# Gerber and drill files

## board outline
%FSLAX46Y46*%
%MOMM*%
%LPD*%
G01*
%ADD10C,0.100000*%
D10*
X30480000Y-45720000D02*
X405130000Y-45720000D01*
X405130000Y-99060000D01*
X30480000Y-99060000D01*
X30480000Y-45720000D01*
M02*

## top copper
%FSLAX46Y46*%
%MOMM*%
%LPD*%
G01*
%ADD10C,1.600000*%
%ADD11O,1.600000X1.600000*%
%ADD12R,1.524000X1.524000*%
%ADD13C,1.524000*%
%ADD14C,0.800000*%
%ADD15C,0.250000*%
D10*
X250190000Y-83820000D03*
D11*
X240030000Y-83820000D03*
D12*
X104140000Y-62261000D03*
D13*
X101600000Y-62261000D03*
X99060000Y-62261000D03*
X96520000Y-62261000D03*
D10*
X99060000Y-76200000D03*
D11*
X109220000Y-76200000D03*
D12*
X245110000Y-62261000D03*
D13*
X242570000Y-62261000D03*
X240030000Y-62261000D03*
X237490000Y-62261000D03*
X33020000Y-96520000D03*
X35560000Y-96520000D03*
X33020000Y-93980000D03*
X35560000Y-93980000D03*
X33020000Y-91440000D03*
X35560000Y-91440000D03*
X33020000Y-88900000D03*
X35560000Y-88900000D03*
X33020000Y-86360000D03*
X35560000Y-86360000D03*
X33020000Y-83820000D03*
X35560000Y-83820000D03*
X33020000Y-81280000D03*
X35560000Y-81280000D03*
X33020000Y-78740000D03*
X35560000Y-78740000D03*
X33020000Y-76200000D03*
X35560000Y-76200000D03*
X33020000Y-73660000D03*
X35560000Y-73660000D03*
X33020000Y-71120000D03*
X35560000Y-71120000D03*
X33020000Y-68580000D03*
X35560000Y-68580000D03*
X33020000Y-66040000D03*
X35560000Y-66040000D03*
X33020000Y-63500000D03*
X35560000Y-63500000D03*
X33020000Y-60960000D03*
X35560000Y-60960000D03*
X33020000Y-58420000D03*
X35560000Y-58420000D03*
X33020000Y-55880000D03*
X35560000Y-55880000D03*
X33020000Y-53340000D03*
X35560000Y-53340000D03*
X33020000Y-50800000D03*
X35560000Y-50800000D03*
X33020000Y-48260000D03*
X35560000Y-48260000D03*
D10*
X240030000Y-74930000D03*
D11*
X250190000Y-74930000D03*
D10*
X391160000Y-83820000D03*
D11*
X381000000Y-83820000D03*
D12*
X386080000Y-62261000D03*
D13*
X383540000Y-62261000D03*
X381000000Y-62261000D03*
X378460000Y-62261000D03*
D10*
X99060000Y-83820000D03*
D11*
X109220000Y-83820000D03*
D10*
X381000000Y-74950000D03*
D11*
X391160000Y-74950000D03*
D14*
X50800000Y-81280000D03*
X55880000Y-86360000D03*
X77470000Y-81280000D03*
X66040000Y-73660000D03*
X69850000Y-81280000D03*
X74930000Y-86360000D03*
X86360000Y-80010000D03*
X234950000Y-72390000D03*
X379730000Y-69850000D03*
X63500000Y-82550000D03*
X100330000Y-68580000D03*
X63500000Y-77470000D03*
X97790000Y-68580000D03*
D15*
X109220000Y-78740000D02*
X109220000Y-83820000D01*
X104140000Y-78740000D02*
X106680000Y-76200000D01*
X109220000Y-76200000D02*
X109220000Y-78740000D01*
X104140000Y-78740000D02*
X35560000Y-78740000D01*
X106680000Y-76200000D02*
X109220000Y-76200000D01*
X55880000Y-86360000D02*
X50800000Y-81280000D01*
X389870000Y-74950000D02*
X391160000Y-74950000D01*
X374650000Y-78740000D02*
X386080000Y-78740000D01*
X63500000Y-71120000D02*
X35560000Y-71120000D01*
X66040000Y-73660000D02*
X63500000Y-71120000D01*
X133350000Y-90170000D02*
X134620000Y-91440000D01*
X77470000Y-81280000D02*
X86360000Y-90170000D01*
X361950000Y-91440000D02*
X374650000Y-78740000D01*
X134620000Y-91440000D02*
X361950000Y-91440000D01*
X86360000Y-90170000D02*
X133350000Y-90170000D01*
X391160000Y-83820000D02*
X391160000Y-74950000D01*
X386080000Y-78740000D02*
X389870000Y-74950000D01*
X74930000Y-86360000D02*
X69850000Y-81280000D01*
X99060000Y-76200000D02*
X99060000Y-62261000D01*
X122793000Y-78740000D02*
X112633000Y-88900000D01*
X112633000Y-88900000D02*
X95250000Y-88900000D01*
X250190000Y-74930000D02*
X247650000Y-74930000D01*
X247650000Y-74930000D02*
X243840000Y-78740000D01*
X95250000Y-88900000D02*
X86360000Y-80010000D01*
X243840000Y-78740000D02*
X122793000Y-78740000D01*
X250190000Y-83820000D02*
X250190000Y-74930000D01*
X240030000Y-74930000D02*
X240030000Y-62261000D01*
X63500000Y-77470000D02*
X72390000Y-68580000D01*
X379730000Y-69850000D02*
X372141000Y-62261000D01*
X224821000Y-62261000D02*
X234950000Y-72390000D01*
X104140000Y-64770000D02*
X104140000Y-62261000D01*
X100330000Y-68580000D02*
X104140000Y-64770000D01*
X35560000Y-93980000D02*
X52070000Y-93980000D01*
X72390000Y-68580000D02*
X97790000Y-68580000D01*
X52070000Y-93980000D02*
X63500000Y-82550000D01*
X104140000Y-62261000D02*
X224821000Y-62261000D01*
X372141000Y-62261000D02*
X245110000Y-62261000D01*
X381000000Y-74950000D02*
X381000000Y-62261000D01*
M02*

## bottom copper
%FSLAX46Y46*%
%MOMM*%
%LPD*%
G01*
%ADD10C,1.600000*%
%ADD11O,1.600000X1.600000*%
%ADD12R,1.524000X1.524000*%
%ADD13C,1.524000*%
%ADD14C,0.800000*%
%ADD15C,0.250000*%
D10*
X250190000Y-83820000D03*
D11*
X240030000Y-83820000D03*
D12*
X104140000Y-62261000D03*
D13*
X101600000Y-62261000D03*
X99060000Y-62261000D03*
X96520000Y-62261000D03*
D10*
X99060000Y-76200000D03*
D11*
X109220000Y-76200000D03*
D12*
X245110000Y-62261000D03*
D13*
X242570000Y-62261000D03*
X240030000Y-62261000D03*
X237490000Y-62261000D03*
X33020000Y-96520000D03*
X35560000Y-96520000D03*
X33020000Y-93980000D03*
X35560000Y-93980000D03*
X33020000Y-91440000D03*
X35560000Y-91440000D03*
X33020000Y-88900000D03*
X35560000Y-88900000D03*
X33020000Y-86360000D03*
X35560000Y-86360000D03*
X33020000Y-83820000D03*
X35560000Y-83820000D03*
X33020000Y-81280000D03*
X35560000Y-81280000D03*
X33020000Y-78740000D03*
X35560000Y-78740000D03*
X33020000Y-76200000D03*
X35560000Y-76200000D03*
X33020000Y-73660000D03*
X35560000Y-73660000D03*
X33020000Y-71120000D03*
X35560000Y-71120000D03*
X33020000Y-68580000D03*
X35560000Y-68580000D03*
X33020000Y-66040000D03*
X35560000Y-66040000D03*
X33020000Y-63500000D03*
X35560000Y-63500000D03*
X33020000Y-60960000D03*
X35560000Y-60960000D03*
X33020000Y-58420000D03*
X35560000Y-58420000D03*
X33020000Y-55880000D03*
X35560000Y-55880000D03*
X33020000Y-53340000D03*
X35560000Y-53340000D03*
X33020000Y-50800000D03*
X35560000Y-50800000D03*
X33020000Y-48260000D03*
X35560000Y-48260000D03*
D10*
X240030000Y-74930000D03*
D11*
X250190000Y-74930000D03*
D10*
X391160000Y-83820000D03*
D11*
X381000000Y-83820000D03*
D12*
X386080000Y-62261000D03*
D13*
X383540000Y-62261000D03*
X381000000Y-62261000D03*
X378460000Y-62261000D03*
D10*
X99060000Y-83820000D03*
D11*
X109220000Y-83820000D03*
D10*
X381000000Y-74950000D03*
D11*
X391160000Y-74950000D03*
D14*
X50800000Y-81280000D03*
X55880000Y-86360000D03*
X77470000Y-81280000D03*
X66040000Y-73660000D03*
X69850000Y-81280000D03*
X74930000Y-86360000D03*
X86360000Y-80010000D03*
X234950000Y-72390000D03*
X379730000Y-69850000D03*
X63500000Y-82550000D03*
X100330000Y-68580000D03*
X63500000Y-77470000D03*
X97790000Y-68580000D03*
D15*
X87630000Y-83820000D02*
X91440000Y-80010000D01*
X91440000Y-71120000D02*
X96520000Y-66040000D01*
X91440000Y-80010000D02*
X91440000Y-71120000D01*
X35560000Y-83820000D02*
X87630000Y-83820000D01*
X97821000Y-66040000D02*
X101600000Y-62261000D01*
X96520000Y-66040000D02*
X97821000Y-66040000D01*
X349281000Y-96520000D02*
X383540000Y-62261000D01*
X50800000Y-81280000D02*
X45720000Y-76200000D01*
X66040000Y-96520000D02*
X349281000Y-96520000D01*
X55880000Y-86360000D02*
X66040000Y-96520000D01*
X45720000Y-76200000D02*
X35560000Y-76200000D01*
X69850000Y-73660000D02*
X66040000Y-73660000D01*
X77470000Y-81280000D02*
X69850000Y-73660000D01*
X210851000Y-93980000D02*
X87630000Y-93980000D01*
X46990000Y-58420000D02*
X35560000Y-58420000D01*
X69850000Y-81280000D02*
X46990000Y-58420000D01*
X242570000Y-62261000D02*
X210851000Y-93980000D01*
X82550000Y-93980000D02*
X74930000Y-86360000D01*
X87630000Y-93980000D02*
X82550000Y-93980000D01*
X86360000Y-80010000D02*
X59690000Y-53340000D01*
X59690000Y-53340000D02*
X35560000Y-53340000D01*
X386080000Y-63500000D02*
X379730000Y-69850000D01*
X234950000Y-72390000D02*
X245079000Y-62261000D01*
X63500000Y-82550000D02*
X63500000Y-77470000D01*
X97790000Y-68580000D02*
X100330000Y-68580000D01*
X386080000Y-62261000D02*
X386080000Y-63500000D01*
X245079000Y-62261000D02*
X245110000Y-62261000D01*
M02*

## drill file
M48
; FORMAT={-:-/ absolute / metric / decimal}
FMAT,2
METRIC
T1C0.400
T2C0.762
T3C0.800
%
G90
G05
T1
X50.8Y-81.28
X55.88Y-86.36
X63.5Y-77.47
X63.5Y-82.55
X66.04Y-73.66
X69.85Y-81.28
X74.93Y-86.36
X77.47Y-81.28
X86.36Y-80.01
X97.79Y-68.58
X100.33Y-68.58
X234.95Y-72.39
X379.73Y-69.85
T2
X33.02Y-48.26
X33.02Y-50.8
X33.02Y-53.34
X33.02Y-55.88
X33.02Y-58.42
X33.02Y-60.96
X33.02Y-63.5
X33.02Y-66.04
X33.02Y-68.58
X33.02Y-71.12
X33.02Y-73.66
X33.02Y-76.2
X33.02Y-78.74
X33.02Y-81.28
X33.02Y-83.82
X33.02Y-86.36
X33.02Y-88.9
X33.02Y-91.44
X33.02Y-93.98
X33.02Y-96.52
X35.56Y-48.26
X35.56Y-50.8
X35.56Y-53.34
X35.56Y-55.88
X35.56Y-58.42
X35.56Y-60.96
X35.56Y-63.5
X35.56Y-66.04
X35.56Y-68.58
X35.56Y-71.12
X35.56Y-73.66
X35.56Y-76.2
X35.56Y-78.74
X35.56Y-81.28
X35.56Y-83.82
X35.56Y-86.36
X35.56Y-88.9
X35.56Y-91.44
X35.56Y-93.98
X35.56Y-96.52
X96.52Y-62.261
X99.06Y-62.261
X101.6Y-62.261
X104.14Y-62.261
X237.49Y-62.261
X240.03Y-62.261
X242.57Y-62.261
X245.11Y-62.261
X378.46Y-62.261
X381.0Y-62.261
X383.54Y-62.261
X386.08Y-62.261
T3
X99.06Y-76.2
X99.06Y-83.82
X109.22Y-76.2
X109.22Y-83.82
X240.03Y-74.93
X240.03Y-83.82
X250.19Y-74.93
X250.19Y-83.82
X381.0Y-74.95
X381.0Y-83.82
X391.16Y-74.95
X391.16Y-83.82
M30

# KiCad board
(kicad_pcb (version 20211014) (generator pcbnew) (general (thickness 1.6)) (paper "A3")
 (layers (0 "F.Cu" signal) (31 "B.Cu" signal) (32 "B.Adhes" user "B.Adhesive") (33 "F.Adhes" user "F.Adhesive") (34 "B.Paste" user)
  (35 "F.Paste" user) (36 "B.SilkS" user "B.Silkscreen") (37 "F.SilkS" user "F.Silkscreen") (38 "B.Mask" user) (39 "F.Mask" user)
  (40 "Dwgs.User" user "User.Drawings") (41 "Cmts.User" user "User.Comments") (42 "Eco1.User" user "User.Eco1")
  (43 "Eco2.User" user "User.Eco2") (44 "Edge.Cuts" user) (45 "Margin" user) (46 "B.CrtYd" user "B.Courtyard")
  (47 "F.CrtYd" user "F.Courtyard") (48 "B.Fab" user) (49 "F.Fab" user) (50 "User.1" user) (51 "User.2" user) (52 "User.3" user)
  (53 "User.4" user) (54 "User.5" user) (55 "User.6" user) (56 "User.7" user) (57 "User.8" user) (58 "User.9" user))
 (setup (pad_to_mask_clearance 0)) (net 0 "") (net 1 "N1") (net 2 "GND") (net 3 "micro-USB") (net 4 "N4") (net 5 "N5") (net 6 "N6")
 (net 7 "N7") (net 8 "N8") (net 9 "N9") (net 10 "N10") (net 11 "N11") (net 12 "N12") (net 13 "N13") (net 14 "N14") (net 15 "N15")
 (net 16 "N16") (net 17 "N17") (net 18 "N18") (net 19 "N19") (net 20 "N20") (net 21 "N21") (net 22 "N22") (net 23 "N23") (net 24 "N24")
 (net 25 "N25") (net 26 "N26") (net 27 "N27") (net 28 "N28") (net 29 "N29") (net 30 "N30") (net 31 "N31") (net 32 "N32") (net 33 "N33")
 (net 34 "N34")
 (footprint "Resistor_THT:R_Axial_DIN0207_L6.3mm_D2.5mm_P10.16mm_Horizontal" (layer "F.Cu") (at 250.19 83.82 180)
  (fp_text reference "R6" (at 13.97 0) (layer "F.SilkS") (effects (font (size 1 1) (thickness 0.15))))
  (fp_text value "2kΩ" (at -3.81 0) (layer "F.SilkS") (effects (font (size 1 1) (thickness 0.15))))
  (pad "1" thru_hole circle (at 0 0 180) (size 1.6 1.6) (drill 0.8) (layers *.Cu *.Mask) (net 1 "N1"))
  (pad "2" thru_hole oval (at 10.16 0 180) (size 1.6 1.6) (drill 0.8) (layers *.Cu *.Mask) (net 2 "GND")))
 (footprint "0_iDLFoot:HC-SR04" (layer "F.Cu") (at 104.14 62.261 180)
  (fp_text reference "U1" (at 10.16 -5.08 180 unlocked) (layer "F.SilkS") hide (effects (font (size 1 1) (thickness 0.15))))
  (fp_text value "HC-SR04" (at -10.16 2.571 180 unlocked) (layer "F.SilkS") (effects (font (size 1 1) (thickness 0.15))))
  (pad "1" thru_hole rect (at 0 0 180) (size 1.524 1.524) (drill 0.762) (layers *.Cu *.Mask) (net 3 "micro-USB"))
  (pad "2" thru_hole circle (at 2.54 0 180) (size 1.524 1.524) (drill 0.762) (layers *.Cu *.Mask) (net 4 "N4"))
  (pad "3" thru_hole circle (at 5.08 0 180) (size 1.524 1.524) (drill 0.762) (layers *.Cu *.Mask) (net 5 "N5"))
  (pad "4" thru_hole circle (at 7.62 0 180) (size 1.524 1.524) (drill 0.762) (layers *.Cu *.Mask) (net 2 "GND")))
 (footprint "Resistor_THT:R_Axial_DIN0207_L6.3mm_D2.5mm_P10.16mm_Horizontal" (layer "F.Cu") (at 99.06 76.2)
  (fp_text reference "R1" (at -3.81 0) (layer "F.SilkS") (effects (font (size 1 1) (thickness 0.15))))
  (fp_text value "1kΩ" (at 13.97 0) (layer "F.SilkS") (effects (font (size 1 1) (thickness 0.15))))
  (pad "1" thru_hole circle (at 0 0) (size 1.6 1.6) (drill 0.8) (layers *.Cu *.Mask) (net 5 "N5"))
  (pad "2" thru_hole oval (at 10.16 0) (size 1.6 1.6) (drill 0.8) (layers *.Cu *.Mask) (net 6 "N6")))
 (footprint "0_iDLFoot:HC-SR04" (layer "F.Cu") (at 245.11 62.261 180)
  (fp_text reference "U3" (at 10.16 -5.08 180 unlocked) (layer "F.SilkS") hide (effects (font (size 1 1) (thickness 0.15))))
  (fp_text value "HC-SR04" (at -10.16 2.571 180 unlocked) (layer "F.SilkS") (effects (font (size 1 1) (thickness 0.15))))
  (pad "1" thru_hole rect (at 0 0 180) (size 1.524 1.524) (drill 0.762) (layers *.Cu *.Mask) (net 3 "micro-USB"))
  (pad "2" thru_hole circle (at 2.54 0 180) (size 1.524 1.524) (drill 0.762) (layers *.Cu *.Mask) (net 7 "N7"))
  (pad "3" thru_hole circle (at 5.08 0 180) (size 1.524 1.524) (drill 0.762) (layers *.Cu *.Mask) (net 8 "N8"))
  (pad "4" thru_hole circle (at 7.62 0 180) (size 1.524 1.524) (drill 0.762) (layers *.Cu *.Mask) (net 2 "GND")))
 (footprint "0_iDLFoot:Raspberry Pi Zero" (layer "F.Cu") (at 33.02 96.52)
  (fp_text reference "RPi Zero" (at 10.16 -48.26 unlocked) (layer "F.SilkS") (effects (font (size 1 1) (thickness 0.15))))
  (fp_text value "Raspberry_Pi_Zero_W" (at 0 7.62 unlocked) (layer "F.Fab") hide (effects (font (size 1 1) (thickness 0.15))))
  (pad "1" thru_hole circle (at 0 0) (size 1.524 1.524) (drill 0.762) (layers *.Cu *.Mask) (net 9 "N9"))
  (pad "2" thru_hole circle (at 2.54 0) (size 1.524 1.524) (drill 0.762) (layers *.Cu *.Mask))
  (pad "3" thru_hole circle (at 0 -2.54) (size 1.524 1.524) (drill 0.762) (layers *.Cu *.Mask) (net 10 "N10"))
  (pad "4" thru_hole circle (at 2.54 -2.54) (size 1.524 1.524) (drill 0.762) (layers *.Cu *.Mask) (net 3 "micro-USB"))
  (pad "5" thru_hole circle (at 0 -5.08) (size 1.524 1.524) (drill 0.762) (layers *.Cu *.Mask) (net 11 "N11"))
  (pad "6" thru_hole circle (at 2.54 -5.08) (size 1.524 1.524) (drill 0.762) (layers *.Cu *.Mask))
  (pad "7" thru_hole circle (at 0 -7.62) (size 1.524 1.524) (drill 0.762) (layers *.Cu *.Mask) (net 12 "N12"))
  (pad "8" thru_hole circle (at 2.54 -7.62) (size 1.524 1.524) (drill 0.762) (layers *.Cu *.Mask) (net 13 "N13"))
  (pad "9" thru_hole circle (at 0 -10.16) (size 1.524 1.524) (drill 0.762) (layers *.Cu *.Mask))
  (pad "10" thru_hole circle (at 2.54 -10.16) (size 1.524 1.524) (drill 0.762) (layers *.Cu *.Mask) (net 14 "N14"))
  (pad "11" thru_hole circle (at 0 -12.7) (size 1.524 1.524) (drill 0.762) (layers *.Cu *.Mask) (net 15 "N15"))
  (pad "12" thru_hole circle (at 2.54 -12.7) (size 1.524 1.524) (drill 0.762) (layers *.Cu *.Mask) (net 4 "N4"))
  (pad "13" thru_hole circle (at 0 -15.24) (size 1.524 1.524) (drill 0.762) (layers *.Cu *.Mask) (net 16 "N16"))
  (pad "14" thru_hole circle (at 2.54 -15.24) (size 1.524 1.524) (drill 0.762) (layers *.Cu *.Mask) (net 2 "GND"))
  (pad "15" thru_hole circle (at 0 -17.78) (size 1.524 1.524) (drill 0.762) (layers *.Cu *.Mask) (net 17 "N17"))
  (pad "16" thru_hole circle (at 2.54 -17.78) (size 1.524 1.524) (drill 0.762) (layers *.Cu *.Mask) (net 6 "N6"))
  (pad "17" thru_hole circle (at 0 -20.32) (size 1.524 1.524) (drill 0.762) (layers *.Cu *.Mask))
  (pad "18" thru_hole circle (at 2.54 -20.32) (size 1.524 1.524) (drill 0.762) (layers *.Cu *.Mask) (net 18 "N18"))
  (pad "19" thru_hole circle (at 0 -22.86) (size 1.524 1.524) (drill 0.762) (layers *.Cu *.Mask) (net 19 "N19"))
  (pad "20" thru_hole circle (at 2.54 -22.86) (size 1.524 1.524) (drill 0.762) (layers *.Cu *.Mask))
  (pad "21" thru_hole circle (at 0 -25.4) (size 1.524 1.524) (drill 0.762) (layers *.Cu *.Mask) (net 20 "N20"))
  (pad "22" thru_hole circle (at 2.54 -25.4) (size 1.524 1.524) (drill 0.762) (layers *.Cu *.Mask) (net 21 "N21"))
  (pad "23" thru_hole circle (at 0 -27.94) (size 1.524 1.524) (drill 0.762) (layers *.Cu *.Mask) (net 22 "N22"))
  (pad "24" thru_hole circle (at 2.54 -27.94) (size 1.524 1.524) (drill 0.762) (layers *.Cu *.Mask) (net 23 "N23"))
  (pad "25" thru_hole circle (at 0 -30.48) (size 1.524 1.524) (drill 0.762) (layers *.Cu *.Mask))
  (pad "26" thru_hole circle (at 2.54 -30.48) (size 1.524 1.524) (drill 0.762) (layers *.Cu *.Mask) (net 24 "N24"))
  (pad "27" thru_hole circle (at 0 -33.02) (size 1.524 1.524) (drill 0.762) (layers *.Cu *.Mask) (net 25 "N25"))
  (pad "28" thru_hole circle (at 2.54 -33.02) (size 1.524 1.524) (drill 0.762) (layers *.Cu *.Mask) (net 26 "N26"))
  (pad "29" thru_hole circle (at 0 -35.56) (size 1.524 1.524) (drill 0.762) (layers *.Cu *.Mask) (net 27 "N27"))
  (pad "30" thru_hole circle (at 2.54 -35.56) (size 1.524 1.524) (drill 0.762) (layers *.Cu *.Mask))
  (pad "31" thru_hole circle (at 0 -38.1) (size 1.524 1.524) (drill 0.762) (layers *.Cu *.Mask) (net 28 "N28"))
  (pad "32" thru_hole circle (at 2.54 -38.1) (size 1.524 1.524) (drill 0.762) (layers *.Cu *.Mask) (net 7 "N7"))
  (pad "33" thru_hole circle (at 0 -40.64) (size 1.524 1.524) (drill 0.762) (layers *.Cu *.Mask) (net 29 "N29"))
  (pad "34" thru_hole circle (at 2.54 -40.64) (size 1.524 1.524) (drill 0.762) (layers *.Cu *.Mask))
  (pad "35" thru_hole circle (at 0 -43.18) (size 1.524 1.524) (drill 0.762) (layers *.Cu *.Mask) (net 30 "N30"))
  (pad "36" thru_hole circle (at 2.54 -43.18) (size 1.524 1.524) (drill 0.762) (layers *.Cu *.Mask) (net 1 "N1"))
  (pad "37" thru_hole circle (at 0 -45.72) (size 1.524 1.524) (drill 0.762) (layers *.Cu *.Mask) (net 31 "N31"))
  (pad "38" thru_hole circle (at 2.54 -45.72) (size 1.524 1.524) (drill 0.762) (layers *.Cu *.Mask) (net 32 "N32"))
  (pad "39" thru_hole circle (at 0 -48.26) (size 1.524 1.524) (drill 0.762) (layers *.Cu *.Mask))
  (pad "40" thru_hole circle (at 2.54 -48.26) (size 1.524 1.524) (drill 0.762) (layers *.Cu *.Mask) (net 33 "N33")))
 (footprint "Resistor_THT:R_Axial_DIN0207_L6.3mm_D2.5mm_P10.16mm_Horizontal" (layer "F.Cu") (at 240.03 74.93)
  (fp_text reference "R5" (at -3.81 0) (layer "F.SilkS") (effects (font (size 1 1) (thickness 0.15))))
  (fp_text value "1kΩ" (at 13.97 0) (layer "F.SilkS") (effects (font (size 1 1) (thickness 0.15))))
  (pad "1" thru_hole circle (at 0 0) (size 1.6 1.6) (drill 0.8) (layers *.Cu *.Mask) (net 8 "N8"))
  (pad "2" thru_hole oval (at 10.16 0) (size 1.6 1.6) (drill 0.8) (layers *.Cu *.Mask) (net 1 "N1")))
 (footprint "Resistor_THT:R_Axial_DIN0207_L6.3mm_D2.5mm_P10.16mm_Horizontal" (layer "F.Cu") (at 391.16 83.82 180)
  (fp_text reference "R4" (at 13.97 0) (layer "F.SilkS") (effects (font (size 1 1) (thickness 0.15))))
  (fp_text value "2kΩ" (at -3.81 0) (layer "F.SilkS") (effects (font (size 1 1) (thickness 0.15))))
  (pad "1" thru_hole circle (at 0 0 180) (size 1.6 1.6) (drill 0.8) (layers *.Cu *.Mask) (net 21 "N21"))
  (pad "2" thru_hole oval (at 10.16 0 180) (size 1.6 1.6) (drill 0.8) (layers *.Cu *.Mask) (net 2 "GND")))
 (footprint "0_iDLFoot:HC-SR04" (layer "F.Cu") (at 386.08 62.261 180)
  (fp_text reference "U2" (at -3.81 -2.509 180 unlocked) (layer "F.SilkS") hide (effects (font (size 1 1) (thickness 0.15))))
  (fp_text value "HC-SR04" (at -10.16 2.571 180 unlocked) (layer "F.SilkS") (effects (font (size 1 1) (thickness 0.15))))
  (pad "1" thru_hole rect (at 0 0 180) (size 1.524 1.524) (drill 0.762) (layers *.Cu *.Mask) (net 3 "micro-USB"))
  (pad "2" thru_hole circle (at 2.54 0 180) (size 1.524 1.524) (drill 0.762) (layers *.Cu *.Mask) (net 18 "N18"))
  (pad "3" thru_hole circle (at 5.08 0 180) (size 1.524 1.524) (drill 0.762) (layers *.Cu *.Mask) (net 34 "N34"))
  (pad "4" thru_hole circle (at 7.62 0 180) (size 1.524 1.524) (drill 0.762) (layers *.Cu *.Mask) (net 2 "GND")))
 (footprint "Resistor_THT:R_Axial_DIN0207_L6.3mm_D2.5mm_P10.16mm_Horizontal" (layer "F.Cu") (at 99.06 83.82)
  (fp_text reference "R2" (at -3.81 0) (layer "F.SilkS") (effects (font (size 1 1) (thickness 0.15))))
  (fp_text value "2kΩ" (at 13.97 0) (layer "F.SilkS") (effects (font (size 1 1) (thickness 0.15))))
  (pad "1" thru_hole circle (at 0 0) (size 1.6 1.6) (drill 0.8) (layers *.Cu *.Mask) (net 2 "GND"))
  (pad "2" thru_hole oval (at 10.16 0) (size 1.6 1.6) (drill 0.8) (layers *.Cu *.Mask) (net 6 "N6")))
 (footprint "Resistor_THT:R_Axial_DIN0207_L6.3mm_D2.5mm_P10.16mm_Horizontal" (layer "F.Cu") (at 381 74.95)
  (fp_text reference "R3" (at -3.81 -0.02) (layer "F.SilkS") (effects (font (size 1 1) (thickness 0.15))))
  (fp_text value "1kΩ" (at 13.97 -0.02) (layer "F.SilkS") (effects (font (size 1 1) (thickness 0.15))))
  (pad "1" thru_hole circle (at 0 0) (size 1.6 1.6) (drill 0.8) (layers *.Cu *.Mask) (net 34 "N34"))
  (pad "2" thru_hole oval (at 10.16 0) (size 1.6 1.6) (drill 0.8) (layers *.Cu *.Mask) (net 21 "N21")))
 (gr_rect (start 30.48 45.72) (end 405.13 99.06) (layer "Edge.Cuts") (width 0.1) (fill none))
 (segment (start 87.63 83.82) (end 91.44 80.01) (width 0.25) (layer "B.Cu") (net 4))
 (segment (start 91.44 71.12) (end 96.52 66.04) (width 0.25) (layer "B.Cu") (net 4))
 (segment (start 91.44 80.01) (end 91.44 71.12) (width 0.25) (layer "B.Cu") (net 4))
 (segment (start 35.56 83.82) (end 87.63 83.82) (width 0.25) (layer "B.Cu") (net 4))
 (segment (start 97.821 66.04) (end 101.6 62.261) (width 0.25) (layer "B.Cu") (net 4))
 (segment (start 96.52 66.04) (end 97.821 66.04) (width 0.25) (layer "B.Cu") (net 4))
 (segment (start 109.22 78.74) (end 109.22 83.82) (width 0.25) (layer "F.Cu") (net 6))
 (segment (start 104.14 78.74) (end 106.68 76.2) (width 0.25) (layer "F.Cu") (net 6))
 (segment (start 109.22 76.2) (end 109.22 78.74) (width 0.25) (layer "F.Cu") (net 6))
 (segment (start 104.14 78.74) (end 35.56 78.74) (width 0.25) (layer "F.Cu") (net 6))
 (segment (start 106.68 76.2) (end 109.22 76.2) (width 0.25) (layer "F.Cu") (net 6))
 (segment (start 55.88 86.36) (end 50.8 81.28) (width 0.25) (layer "F.Cu") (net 18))
 (via (at 50.8 81.28) (size 0.8) (drill 0.4) (layers "F.Cu" "B.Cu") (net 18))
 (via (at 55.88 86.36) (size 0.8) (drill 0.4) (layers "F.Cu" "B.Cu") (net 18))
 (segment (start 349.281 96.52) (end 383.54 62.261) (width 0.25) (layer "B.Cu") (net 18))
 (segment (start 50.8 81.28) (end 45.72 76.2) (width 0.25) (layer "B.Cu") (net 18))
 (segment (start 66.04 96.52) (end 349.281 96.52) (width 0.25) (layer "B.Cu") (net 18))
 (segment (start 55.88 86.36) (end 66.04 96.52) (width 0.25) (layer "B.Cu") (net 18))
 (segment (start 45.72 76.2) (end 35.56 76.2) (width 0.25) (layer "B.Cu") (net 18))
 (segment (start 389.87 74.95) (end 391.16 74.95) (width 0.25) (layer "F.Cu") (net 21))
 (segment (start 374.65 78.74) (end 386.08 78.74) (width 0.25) (layer "F.Cu") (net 21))
 (segment (start 63.5 71.12) (end 35.56 71.12) (width 0.25) (layer "F.Cu") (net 21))
 (segment (start 66.04 73.66) (end 63.5 71.12) (width 0.25) (layer "F.Cu") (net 21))
 (segment (start 133.35 90.17) (end 134.62 91.44) (width 0.25) (layer "F.Cu") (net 21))
 (segment (start 77.47 81.28) (end 86.36 90.17) (width 0.25) (layer "F.Cu") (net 21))
 (segment (start 361.95 91.44) (end 374.65 78.74) (width 0.25) (layer "F.Cu") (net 21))
 (segment (start 134.62 91.44) (end 361.95 91.44) (width 0.25) (layer "F.Cu") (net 21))
 (segment (start 86.36 90.17) (end 133.35 90.17) (width 0.25) (layer "F.Cu") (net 21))
 (segment (start 391.16 83.82) (end 391.16 74.95) (width 0.25) (layer "F.Cu") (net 21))
 (segment (start 386.08 78.74) (end 389.87 74.95) (width 0.25) (layer "F.Cu") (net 21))
 (via (at 77.47 81.28) (size 0.8) (drill 0.4) (layers "F.Cu" "B.Cu") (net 21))
 (via (at 66.04 73.66) (size 0.8) (drill 0.4) (layers "F.Cu" "B.Cu") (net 21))
 (segment (start 69.85 73.66) (end 66.04 73.66) (width 0.25) (layer "B.Cu") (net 21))
 (segment (start 77.47 81.28) (end 69.85 73.66) (width 0.25) (layer "B.Cu") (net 21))
 (segment (start 74.93 86.36) (end 69.85 81.28) (width 0.25) (layer "F.Cu") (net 7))
 (via (at 69.85 81.28) (size 0.8) (drill 0.4) (layers "F.Cu" "B.Cu") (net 7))
 (via (at 74.93 86.36) (size 0.8) (drill 0.4) (layers "F.Cu" "B.Cu") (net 7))
 (segment (start 210.851 93.98) (end 87.63 93.98) (width 0.25) (layer "B.Cu") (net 7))
 (segment (start 46.99 58.42) (end 35.56 58.42) (width 0.25) (layer "B.Cu") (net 7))
 (segment (start 69.85 81.28) (end 46.99 58.42) (width 0.25) (layer "B.Cu") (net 7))
 (segment (start 242.57 62.261) (end 210.851 93.98) (width 0.25) (layer "B.Cu") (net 7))
 (segment (start 82.55 93.98) (end 74.93 86.36) (width 0.25) (layer "B.Cu") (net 7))
 (segment (start 87.63 93.98) (end 82.55 93.98) (width 0.25) (layer "B.Cu") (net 7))
 (segment (start 99.06 76.2) (end 99.06 62.261) (width 0.25) (layer "F.Cu") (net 5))
 (segment (start 122.793 78.74) (end 112.633 88.9) (width 0.25) (layer "F.Cu") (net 1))
 (segment (start 112.633 88.9) (end 95.25 88.9) (width 0.25) (layer "F.Cu") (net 1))
 (segment (start 250.19 74.93) (end 247.65 74.93) (width 0.25) (layer "F.Cu") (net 1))
 (segment (start 247.65 74.93) (end 243.84 78.74) (width 0.25) (layer "F.Cu") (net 1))
 (segment (start 95.25 88.9) (end 86.36 80.01) (width 0.25) (layer "F.Cu") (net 1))
 (segment (start 243.84 78.74) (end 122.793 78.74) (width 0.25) (layer "F.Cu") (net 1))
 (segment (start 250.19 83.82) (end 250.19 74.93) (width 0.25) (layer "F.Cu") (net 1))
 (via (at 86.36 80.01) (size 0.8) (drill 0.4) (layers "F.Cu" "B.Cu") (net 1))
 (segment (start 86.36 80.01) (end 59.69 53.34) (width 0.25) (layer "B.Cu") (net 1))
 (segment (start 59.69 53.34) (end 35.56 53.34) (width 0.25) (layer "B.Cu") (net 1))
 (segment (start 240.03 74.93) (end 240.03 62.261) (width 0.25) (layer "F.Cu") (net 8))
 (segment (start 63.5 77.47) (end 72.39 68.58) (width 0.25) (layer "F.Cu") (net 3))
 (segment (start 379.73 69.85) (end 372.141 62.261) (width 0.25) (layer "F.Cu") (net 3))
 (segment (start 224.821 62.261) (end 234.95 72.39) (width 0.25) (layer "F.Cu") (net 3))
 (segment (start 104.14 64.77) (end 104.14 62.261) (width 0.25) (layer "F.Cu") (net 3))
 (segment (start 100.33 68.58) (end 104.14 64.77) (width 0.25) (layer "F.Cu") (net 3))
 (segment (start 35.56 93.98) (end 52.07 93.98) (width 0.25) (layer "F.Cu") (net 3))
 (segment (start 72.39 68.58) (end 97.79 68.58) (width 0.25) (layer "F.Cu") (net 3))
 (segment (start 52.07 93.98) (end 63.5 82.55) (width 0.25) (layer "F.Cu") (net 3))
 (segment (start 104.14 62.261) (end 224.821 62.261) (width 0.25) (layer "F.Cu") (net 3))
 (segment (start 372.141 62.261) (end 245.11 62.261) (width 0.25) (layer "F.Cu") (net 3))
 (via (at 234.95 72.39) (size 0.8) (drill 0.4) (layers "F.Cu" "B.Cu") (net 3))
 (via (at 379.73 69.85) (size 0.8) (drill 0.4) (layers "F.Cu" "B.Cu") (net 3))
 (via (at 63.5 82.55) (size 0.8) (drill 0.4) (layers "F.Cu" "B.Cu") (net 3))
 (via (at 100.33 68.58) (size 0.8) (drill 0.4) (layers "F.Cu" "B.Cu") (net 3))
 (via (at 63.5 77.47) (size 0.8) (drill 0.4) (layers "F.Cu" "B.Cu") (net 3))
 (via (at 97.79 68.58) (size 0.8) (drill 0.4) (layers "F.Cu" "B.Cu") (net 3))
 (segment (start 386.08 63.5) (end 379.73 69.85) (width 0.25) (layer "B.Cu") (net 3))
 (segment (start 234.95 72.39) (end 245.079 62.261) (width 0.25) (layer "B.Cu") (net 3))
 (segment (start 63.5 82.55) (end 63.5 77.47) (width 0.25) (layer "B.Cu") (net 3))
 (segment (start 97.79 68.58) (end 100.33 68.58) (width 0.25) (layer "B.Cu") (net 3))
 (segment (start 386.08 62.261) (end 386.08 63.5) (width 0.25) (layer "B.Cu") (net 3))
 (segment (start 245.079 62.261) (end 245.11 62.261) (width 0.25) (layer "B.Cu") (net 3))
 (segment (start 381 74.95) (end 381 62.261) (width 0.25) (layer "F.Cu") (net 34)))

